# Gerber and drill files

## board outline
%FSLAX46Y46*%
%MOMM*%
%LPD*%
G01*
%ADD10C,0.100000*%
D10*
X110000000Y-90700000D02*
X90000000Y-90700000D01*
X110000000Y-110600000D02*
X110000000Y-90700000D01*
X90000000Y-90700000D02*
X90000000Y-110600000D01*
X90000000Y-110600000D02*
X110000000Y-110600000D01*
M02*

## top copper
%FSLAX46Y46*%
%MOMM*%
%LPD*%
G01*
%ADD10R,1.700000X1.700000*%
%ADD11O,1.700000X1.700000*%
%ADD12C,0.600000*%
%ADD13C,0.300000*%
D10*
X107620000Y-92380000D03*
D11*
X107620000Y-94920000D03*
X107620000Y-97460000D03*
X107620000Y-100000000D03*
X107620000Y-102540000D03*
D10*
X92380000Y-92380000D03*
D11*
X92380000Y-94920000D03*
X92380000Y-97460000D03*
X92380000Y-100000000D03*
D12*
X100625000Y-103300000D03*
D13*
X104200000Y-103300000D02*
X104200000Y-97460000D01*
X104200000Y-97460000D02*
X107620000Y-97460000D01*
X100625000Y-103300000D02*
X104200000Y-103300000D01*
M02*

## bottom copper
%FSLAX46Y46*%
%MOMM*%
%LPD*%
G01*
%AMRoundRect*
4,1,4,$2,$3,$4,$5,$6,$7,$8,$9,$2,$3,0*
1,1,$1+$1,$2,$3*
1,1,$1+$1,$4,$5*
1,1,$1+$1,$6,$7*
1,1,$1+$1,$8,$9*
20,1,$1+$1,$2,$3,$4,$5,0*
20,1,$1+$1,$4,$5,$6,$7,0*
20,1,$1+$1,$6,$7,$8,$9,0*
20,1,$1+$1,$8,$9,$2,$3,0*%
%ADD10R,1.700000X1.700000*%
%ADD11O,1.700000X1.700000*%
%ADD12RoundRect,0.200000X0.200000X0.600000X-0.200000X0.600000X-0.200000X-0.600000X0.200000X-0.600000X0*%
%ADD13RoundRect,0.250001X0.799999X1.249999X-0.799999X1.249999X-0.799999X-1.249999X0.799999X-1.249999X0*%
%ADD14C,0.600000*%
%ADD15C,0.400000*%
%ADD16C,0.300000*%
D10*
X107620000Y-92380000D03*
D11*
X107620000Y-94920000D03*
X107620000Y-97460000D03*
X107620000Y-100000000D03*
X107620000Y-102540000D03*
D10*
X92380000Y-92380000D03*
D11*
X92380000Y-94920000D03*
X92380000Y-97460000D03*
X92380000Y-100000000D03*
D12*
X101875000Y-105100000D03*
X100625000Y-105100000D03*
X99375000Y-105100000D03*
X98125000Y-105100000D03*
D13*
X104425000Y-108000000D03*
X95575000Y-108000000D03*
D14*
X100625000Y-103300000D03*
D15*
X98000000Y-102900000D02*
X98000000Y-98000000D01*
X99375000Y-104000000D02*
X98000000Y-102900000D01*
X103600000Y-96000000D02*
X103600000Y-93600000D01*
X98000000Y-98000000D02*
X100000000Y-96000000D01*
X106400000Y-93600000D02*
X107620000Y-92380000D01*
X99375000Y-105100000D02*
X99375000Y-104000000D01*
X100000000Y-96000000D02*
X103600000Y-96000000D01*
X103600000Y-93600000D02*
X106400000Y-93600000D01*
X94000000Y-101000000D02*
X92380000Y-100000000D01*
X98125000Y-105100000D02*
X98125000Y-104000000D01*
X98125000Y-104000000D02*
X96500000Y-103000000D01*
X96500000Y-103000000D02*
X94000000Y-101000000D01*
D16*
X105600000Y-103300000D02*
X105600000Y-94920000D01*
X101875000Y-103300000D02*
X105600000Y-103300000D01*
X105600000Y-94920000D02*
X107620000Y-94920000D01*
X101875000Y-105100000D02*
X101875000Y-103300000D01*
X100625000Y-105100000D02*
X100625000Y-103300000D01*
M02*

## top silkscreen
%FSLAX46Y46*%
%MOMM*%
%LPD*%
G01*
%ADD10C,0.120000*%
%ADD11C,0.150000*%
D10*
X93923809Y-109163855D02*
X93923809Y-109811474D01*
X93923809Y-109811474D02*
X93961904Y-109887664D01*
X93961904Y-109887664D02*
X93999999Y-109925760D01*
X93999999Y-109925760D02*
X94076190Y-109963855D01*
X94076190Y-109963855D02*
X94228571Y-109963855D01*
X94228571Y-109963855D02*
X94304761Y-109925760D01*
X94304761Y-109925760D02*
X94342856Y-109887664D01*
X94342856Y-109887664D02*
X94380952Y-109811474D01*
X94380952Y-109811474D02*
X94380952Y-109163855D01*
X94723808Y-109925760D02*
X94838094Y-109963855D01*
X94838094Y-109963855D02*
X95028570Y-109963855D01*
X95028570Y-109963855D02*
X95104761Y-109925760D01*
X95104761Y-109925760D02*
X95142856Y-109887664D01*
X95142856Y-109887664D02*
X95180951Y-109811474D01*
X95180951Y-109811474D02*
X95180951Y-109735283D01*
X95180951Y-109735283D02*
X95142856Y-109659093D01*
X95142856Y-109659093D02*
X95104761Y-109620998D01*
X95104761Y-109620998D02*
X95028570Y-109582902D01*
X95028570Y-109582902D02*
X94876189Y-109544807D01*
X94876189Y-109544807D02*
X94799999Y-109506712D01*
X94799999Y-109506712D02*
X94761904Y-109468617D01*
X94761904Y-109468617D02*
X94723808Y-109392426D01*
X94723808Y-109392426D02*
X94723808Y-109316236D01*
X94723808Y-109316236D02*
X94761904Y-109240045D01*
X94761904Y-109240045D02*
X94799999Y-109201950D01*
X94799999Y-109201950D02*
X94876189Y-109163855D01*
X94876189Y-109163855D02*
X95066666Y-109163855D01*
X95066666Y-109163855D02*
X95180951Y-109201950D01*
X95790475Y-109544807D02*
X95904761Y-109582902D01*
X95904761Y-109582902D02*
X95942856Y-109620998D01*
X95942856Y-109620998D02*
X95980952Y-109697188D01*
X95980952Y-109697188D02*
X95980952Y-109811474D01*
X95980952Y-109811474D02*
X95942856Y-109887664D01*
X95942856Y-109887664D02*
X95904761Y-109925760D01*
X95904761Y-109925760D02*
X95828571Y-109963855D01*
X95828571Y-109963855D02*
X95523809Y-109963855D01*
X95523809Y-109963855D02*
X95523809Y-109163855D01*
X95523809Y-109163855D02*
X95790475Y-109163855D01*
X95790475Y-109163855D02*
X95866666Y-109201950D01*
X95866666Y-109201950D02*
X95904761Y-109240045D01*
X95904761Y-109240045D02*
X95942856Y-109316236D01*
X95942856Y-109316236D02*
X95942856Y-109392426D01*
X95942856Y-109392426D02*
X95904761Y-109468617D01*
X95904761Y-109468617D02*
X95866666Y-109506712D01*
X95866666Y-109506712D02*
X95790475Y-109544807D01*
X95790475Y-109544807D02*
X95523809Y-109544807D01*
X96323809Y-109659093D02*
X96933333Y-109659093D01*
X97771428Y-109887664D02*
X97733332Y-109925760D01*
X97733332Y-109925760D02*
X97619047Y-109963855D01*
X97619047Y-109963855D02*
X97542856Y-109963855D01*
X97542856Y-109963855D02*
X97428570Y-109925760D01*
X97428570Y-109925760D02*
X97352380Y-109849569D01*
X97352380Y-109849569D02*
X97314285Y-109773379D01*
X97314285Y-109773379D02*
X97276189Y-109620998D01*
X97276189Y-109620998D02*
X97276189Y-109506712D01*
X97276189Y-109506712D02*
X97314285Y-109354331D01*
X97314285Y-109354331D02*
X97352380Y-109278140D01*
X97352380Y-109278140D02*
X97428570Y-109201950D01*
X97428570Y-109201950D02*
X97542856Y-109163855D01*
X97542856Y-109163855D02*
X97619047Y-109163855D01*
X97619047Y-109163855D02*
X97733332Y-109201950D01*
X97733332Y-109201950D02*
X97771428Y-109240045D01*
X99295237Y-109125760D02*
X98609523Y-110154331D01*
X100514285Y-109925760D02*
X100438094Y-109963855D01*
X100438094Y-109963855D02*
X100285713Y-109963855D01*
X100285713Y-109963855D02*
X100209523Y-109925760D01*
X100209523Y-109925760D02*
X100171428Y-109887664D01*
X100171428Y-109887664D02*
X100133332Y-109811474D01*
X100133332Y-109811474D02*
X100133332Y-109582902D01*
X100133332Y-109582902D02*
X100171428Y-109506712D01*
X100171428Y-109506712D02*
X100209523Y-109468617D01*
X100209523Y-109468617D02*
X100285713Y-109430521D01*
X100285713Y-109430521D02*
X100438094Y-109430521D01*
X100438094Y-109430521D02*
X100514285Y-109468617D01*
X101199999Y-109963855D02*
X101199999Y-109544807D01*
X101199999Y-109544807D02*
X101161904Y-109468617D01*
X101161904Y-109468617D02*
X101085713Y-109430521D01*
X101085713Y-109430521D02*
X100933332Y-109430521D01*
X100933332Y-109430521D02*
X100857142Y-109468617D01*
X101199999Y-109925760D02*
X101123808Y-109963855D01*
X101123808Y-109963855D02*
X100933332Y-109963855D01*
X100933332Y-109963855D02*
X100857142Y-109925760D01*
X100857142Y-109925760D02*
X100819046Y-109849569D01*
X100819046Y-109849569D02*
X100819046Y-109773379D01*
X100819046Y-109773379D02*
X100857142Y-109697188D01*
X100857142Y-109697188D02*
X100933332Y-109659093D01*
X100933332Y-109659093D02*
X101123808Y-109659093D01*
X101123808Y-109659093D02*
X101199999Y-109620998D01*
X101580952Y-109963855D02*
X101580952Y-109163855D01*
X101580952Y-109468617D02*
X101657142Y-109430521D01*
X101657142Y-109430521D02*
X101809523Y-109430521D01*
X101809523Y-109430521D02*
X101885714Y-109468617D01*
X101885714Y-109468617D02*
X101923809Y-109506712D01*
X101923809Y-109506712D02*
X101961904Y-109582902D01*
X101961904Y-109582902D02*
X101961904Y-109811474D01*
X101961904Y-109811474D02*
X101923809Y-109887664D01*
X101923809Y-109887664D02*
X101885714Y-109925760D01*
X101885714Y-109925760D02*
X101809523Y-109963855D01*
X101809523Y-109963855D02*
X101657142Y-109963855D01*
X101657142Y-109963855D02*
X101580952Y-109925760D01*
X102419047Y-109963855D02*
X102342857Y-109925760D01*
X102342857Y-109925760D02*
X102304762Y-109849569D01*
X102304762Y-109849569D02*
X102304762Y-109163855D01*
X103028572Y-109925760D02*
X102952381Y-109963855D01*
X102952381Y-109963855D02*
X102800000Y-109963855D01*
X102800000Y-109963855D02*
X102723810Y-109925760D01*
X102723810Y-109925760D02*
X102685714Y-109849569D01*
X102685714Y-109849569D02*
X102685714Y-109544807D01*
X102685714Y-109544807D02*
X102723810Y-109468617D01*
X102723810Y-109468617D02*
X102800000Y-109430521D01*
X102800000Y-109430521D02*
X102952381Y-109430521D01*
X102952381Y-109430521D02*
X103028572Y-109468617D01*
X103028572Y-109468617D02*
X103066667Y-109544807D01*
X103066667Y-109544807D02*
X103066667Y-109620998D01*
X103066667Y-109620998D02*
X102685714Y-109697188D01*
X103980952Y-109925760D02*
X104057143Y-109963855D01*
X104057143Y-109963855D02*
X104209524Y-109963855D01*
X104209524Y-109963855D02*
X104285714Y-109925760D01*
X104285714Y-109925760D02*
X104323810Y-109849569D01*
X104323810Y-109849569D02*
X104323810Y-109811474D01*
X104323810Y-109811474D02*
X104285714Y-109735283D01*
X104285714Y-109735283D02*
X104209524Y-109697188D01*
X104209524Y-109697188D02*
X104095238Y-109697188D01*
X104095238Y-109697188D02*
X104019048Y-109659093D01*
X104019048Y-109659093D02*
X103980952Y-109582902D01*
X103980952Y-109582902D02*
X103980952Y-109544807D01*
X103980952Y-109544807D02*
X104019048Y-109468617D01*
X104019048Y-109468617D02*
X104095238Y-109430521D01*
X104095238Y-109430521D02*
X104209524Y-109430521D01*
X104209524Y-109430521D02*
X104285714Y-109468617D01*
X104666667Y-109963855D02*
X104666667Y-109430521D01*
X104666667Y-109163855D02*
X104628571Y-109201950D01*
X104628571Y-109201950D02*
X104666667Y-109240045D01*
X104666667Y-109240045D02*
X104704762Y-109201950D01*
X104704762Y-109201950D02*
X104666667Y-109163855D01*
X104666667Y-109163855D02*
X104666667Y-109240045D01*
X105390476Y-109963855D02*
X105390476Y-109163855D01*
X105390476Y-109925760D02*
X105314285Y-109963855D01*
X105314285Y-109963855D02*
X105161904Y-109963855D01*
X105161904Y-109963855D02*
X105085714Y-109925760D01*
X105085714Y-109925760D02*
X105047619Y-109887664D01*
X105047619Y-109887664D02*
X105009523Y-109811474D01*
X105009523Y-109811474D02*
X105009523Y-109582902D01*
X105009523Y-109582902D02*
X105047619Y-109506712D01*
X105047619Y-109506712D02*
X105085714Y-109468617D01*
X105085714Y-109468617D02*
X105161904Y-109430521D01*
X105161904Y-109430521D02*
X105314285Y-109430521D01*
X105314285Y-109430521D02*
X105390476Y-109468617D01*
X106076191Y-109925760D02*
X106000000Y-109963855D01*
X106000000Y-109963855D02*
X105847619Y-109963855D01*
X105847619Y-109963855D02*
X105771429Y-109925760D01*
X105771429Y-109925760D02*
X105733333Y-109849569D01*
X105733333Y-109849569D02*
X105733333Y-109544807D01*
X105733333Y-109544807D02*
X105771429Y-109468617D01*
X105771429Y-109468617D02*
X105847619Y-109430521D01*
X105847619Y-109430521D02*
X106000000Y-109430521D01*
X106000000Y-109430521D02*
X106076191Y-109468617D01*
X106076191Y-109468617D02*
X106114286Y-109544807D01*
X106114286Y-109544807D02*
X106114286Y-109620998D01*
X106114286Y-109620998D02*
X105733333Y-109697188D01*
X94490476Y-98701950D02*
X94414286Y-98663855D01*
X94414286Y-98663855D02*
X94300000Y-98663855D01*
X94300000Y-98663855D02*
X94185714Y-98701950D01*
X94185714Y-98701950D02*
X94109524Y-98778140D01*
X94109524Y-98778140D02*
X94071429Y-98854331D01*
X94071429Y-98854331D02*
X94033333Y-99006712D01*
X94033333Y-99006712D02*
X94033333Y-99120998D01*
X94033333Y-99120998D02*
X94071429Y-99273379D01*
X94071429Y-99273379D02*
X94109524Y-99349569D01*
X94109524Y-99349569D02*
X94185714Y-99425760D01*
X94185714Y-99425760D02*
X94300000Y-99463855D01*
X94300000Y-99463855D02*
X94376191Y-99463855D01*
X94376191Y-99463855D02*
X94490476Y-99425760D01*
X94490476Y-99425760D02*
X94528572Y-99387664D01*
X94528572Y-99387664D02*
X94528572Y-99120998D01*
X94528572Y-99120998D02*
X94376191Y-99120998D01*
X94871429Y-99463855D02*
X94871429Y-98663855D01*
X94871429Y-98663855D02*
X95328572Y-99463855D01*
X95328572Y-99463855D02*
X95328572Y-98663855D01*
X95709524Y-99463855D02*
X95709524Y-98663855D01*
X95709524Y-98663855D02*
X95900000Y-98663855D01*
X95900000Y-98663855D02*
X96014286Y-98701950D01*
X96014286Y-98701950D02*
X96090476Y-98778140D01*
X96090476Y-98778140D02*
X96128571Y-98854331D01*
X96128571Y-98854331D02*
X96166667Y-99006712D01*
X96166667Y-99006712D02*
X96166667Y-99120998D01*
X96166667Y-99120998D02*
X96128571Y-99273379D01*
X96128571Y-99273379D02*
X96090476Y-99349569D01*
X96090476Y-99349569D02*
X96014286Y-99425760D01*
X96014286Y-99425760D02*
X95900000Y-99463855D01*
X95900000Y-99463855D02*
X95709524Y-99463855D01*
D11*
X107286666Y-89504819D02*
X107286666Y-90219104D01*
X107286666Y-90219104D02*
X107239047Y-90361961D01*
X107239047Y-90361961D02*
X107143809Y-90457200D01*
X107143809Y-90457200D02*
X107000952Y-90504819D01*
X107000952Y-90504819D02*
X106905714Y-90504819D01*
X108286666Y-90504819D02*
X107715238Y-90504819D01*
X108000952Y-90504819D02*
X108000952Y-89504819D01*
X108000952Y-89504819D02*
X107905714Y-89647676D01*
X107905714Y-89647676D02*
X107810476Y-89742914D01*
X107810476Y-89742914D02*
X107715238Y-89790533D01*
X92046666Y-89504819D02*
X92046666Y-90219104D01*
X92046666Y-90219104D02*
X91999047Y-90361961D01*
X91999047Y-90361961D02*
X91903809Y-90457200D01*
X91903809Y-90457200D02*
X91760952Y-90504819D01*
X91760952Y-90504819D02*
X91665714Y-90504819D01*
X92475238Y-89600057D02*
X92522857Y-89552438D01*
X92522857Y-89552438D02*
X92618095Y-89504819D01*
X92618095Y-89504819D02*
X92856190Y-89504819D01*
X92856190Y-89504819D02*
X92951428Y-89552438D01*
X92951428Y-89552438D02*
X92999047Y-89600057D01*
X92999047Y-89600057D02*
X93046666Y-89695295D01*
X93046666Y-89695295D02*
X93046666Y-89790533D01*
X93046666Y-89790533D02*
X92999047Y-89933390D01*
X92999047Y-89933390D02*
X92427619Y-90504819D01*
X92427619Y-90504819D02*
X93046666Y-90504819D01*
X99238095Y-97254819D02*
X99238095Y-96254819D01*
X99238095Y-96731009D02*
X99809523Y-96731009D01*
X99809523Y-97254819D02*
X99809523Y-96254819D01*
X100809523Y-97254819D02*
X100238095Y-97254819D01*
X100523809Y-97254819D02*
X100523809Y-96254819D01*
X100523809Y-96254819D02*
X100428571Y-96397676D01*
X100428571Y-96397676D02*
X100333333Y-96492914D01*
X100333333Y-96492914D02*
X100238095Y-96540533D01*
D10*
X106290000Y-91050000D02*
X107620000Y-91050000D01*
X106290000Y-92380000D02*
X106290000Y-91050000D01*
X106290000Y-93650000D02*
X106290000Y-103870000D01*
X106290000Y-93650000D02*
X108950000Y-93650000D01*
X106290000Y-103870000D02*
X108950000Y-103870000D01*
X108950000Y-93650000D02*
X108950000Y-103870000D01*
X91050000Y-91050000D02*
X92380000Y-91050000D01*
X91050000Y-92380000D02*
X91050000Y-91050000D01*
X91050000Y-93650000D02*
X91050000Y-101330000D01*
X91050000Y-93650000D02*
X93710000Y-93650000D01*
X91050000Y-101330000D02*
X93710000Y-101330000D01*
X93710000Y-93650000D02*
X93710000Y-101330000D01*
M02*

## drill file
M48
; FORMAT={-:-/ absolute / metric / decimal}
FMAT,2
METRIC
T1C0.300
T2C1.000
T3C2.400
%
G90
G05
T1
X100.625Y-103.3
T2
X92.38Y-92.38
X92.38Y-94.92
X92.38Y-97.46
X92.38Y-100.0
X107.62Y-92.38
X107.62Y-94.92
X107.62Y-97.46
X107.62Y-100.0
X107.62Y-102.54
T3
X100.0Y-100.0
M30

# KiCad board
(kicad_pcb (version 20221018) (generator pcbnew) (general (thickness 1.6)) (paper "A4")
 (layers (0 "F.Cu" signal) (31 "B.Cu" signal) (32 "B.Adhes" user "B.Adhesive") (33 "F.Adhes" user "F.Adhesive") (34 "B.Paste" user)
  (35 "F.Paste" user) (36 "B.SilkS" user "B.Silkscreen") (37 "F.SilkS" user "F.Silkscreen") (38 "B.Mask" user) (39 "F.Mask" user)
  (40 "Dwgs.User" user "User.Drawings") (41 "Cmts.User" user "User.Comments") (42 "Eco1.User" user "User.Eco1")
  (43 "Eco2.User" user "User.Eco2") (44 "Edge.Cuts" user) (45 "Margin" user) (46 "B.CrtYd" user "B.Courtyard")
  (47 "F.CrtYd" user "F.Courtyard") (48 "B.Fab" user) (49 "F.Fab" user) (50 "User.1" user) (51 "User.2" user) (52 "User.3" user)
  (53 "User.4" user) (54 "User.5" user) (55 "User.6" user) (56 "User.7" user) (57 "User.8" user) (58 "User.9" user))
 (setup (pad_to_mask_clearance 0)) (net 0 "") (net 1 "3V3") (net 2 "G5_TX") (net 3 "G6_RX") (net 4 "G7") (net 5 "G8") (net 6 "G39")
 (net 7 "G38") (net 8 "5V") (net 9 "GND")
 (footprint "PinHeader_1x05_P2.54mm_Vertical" (layer "F.Cu") (at 107.62 92.38)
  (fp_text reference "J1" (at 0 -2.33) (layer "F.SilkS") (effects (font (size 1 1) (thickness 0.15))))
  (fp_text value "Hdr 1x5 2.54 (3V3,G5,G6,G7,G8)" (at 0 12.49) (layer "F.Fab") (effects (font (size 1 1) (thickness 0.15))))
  (fp_line (start -1.33 -1.33) (end 0 -1.33) (stroke (width 0.12) (type solid)) (layer "F.SilkS"))
  (fp_line (start -1.33 0) (end -1.33 -1.33) (stroke (width 0.12) (type solid)) (layer "F.SilkS"))
  (fp_line (start -1.33 1.27) (end -1.33 11.49) (stroke (width 0.12) (type solid)) (layer "F.SilkS"))
  (fp_line (start -1.33 1.27) (end 1.33 1.27) (stroke (width 0.12) (type solid)) (layer "F.SilkS"))
  (fp_line (start -1.33 11.49) (end 1.33 11.49) (stroke (width 0.12) (type solid)) (layer "F.SilkS"))
  (fp_line (start 1.33 1.27) (end 1.33 11.49) (stroke (width 0.12) (type solid)) (layer "F.SilkS"))
  (pad "1" thru_hole rect (at 0 0) (size 1.7 1.7) (drill 1) (layers "*.Cu" "*.Mask") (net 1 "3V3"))
  (pad "2" thru_hole oval (at 0 2.54) (size 1.7 1.7) (drill 1) (layers "*.Cu" "*.Mask") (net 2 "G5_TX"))
  (pad "3" thru_hole oval (at 0 5.08) (size 1.7 1.7) (drill 1) (layers "*.Cu" "*.Mask") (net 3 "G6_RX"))
  (pad "4" thru_hole oval (at 0 7.62) (size 1.7 1.7) (drill 1) (layers "*.Cu" "*.Mask") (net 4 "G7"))
  (pad "5" thru_hole oval (at 0 10.16) (size 1.7 1.7) (drill 1) (layers "*.Cu" "*.Mask") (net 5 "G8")))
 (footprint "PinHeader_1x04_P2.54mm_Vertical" (layer "F.Cu") (at 92.38 92.38)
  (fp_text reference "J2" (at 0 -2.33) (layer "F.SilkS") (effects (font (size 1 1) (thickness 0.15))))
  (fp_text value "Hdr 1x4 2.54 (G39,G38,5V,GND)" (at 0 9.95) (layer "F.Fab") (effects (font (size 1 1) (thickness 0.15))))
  (fp_line (start -1.33 -1.33) (end 0 -1.33) (stroke (width 0.12) (type solid)) (layer "F.SilkS"))
  (fp_line (start -1.33 0) (end -1.33 -1.33) (stroke (width 0.12) (type solid)) (layer "F.SilkS"))
  (fp_line (start -1.33 1.27) (end -1.33 8.95) (stroke (width 0.12) (type solid)) (layer "F.SilkS"))
  (fp_line (start -1.33 1.27) (end 1.33 1.27) (stroke (width 0.12) (type solid)) (layer "F.SilkS"))
  (fp_line (start -1.33 8.95) (end 1.33 8.95) (stroke (width 0.12) (type solid)) (layer "F.SilkS"))
  (fp_line (start 1.33 1.27) (end 1.33 8.95) (stroke (width 0.12) (type solid)) (layer "F.SilkS"))
  (pad "1" thru_hole rect (at 0 0) (size 1.7 1.7) (drill 1) (layers "*.Cu" "*.Mask") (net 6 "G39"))
  (pad "2" thru_hole oval (at 0 2.54) (size 1.7 1.7) (drill 1) (layers "*.Cu" "*.Mask") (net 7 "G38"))
  (pad "3" thru_hole oval (at 0 5.08) (size 1.7 1.7) (drill 1) (layers "*.Cu" "*.Mask") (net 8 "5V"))
  (pad "4" thru_hole oval (at 0 7.62) (size 1.7 1.7) (drill 1) (layers "*.Cu" "*.Mask") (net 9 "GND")))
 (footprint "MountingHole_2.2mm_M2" (layer "F.Cu") (at 100 100)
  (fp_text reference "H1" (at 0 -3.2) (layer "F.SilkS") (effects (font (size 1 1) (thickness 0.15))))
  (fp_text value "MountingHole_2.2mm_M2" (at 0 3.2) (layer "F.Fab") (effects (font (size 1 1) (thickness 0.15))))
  (pad "" np_thru_hole circle (at 0 0) (size 2.4 2.4) (drill 2.4) (layers "*.Cu" "*.Mask")))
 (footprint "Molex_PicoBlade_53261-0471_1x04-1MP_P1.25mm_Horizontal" (layer "B.Cu") (at 100 107.5 180)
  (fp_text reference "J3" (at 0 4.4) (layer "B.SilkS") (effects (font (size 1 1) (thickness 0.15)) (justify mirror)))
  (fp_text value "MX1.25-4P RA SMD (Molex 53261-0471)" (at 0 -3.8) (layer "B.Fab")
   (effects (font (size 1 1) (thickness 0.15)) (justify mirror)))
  (pad "1" smd roundrect (at -1.875 2.4 180) (size 0.8 1.6) (layers "B.Cu" "B.Paste" "B.Mask") (roundrect_rratio 0.25) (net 2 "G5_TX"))
  (pad "2" smd roundrect (at -0.625 2.4 180) (size 0.8 1.6) (layers "B.Cu" "B.Paste" "B.Mask") (roundrect_rratio 0.25) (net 3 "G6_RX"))
  (pad "3" smd roundrect (at 0.625 2.4 180) (size 0.8 1.6) (layers "B.Cu" "B.Paste" "B.Mask") (roundrect_rratio 0.25) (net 1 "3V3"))
  (pad "4" smd roundrect (at 1.875 2.4 180) (size 0.8 1.6) (layers "B.Cu" "B.Paste" "B.Mask") (roundrect_rratio 0.25) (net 9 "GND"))
  (pad "MP" smd roundrect (at -4.425 -0.5 180) (size 2.1 3) (layers "B.Cu" "B.Paste" "B.Mask") (roundrect_rratio 0.119048))
  (pad "MP" smd roundrect (at 4.425 -0.5 180) (size 2.1 3) (layers "B.Cu" "B.Paste" "B.Mask") (roundrect_rratio 0.119048)))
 (gr_line (start 110 90.7) (end 90 90.7) (stroke (width 0.1) (type default)) (layer "Edge.Cuts"))
 (gr_line (start 110 110.6) (end 110 90.7) (stroke (width 0.1) (type default)) (layer "Edge.Cuts"))
 (gr_line (start 90 90.7) (end 90 110.6) (stroke (width 0.1) (type default)) (layer "Edge.Cuts"))
 (gr_line (start 90 110.6) (end 110 110.6) (stroke (width 0.1) (type default)) (layer "Edge.Cuts"))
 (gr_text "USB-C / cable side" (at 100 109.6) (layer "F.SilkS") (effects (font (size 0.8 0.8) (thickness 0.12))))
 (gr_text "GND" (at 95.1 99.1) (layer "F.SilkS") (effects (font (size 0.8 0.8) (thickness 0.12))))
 (segment (start 98 102.9) (end 98 98) (width 0.4) (layer "B.Cu") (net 1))
 (segment (start 99.375 104) (end 98 102.9) (width 0.4) (layer "B.Cu") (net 1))
 (segment (start 103.6 96) (end 103.6 93.6) (width 0.4) (layer "B.Cu") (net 1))
 (segment (start 98 98) (end 100 96) (width 0.4) (layer "B.Cu") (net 1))
 (segment (start 106.4 93.6) (end 107.62 92.38) (width 0.4) (layer "B.Cu") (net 1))
 (segment (start 99.375 105.1) (end 99.375 104) (width 0.4) (layer "B.Cu") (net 1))
 (segment (start 100 96) (end 103.6 96) (width 0.4) (layer "B.Cu") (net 1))
 (segment (start 103.6 93.6) (end 106.4 93.6) (width 0.4) (layer "B.Cu") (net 1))
 (segment (start 94 101) (end 92.38 100) (width 0.4) (layer "B.Cu") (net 9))
 (segment (start 98.125 105.1) (end 98.125 104) (width 0.4) (layer "B.Cu") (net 9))
 (segment (start 98.125 104) (end 96.5 103) (width 0.4) (layer "B.Cu") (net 9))
 (segment (start 96.5 103) (end 94 101) (width 0.4) (layer "B.Cu") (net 9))
 (segment (start 105.6 103.3) (end 105.6 94.92) (width 0.3) (layer "B.Cu") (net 2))
 (segment (start 101.875 103.3) (end 105.6 103.3) (width 0.3) (layer "B.Cu") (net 2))
 (segment (start 105.6 94.92) (end 107.62 94.92) (width 0.3) (layer "B.Cu") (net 2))
 (segment (start 101.875 105.1) (end 101.875 103.3) (width 0.3) (layer "B.Cu") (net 2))
 (segment (start 104.2 103.3) (end 104.2 97.46) (width 0.3) (layer "F.Cu") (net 3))
 (segment (start 104.2 97.46) (end 107.62 97.46) (width 0.3) (layer "F.Cu") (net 3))
 (segment (start 100.625 103.3) (end 104.2 103.3) (width 0.3) (layer "F.Cu") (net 3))
 (via (at 100.625 103.3) (size 0.6) (drill 0.3) (layers "F.Cu" "B.Cu") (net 3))
 (segment (start 100.625 105.1) (end 100.625 103.3) (width 0.3) (layer "B.Cu") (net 3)))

